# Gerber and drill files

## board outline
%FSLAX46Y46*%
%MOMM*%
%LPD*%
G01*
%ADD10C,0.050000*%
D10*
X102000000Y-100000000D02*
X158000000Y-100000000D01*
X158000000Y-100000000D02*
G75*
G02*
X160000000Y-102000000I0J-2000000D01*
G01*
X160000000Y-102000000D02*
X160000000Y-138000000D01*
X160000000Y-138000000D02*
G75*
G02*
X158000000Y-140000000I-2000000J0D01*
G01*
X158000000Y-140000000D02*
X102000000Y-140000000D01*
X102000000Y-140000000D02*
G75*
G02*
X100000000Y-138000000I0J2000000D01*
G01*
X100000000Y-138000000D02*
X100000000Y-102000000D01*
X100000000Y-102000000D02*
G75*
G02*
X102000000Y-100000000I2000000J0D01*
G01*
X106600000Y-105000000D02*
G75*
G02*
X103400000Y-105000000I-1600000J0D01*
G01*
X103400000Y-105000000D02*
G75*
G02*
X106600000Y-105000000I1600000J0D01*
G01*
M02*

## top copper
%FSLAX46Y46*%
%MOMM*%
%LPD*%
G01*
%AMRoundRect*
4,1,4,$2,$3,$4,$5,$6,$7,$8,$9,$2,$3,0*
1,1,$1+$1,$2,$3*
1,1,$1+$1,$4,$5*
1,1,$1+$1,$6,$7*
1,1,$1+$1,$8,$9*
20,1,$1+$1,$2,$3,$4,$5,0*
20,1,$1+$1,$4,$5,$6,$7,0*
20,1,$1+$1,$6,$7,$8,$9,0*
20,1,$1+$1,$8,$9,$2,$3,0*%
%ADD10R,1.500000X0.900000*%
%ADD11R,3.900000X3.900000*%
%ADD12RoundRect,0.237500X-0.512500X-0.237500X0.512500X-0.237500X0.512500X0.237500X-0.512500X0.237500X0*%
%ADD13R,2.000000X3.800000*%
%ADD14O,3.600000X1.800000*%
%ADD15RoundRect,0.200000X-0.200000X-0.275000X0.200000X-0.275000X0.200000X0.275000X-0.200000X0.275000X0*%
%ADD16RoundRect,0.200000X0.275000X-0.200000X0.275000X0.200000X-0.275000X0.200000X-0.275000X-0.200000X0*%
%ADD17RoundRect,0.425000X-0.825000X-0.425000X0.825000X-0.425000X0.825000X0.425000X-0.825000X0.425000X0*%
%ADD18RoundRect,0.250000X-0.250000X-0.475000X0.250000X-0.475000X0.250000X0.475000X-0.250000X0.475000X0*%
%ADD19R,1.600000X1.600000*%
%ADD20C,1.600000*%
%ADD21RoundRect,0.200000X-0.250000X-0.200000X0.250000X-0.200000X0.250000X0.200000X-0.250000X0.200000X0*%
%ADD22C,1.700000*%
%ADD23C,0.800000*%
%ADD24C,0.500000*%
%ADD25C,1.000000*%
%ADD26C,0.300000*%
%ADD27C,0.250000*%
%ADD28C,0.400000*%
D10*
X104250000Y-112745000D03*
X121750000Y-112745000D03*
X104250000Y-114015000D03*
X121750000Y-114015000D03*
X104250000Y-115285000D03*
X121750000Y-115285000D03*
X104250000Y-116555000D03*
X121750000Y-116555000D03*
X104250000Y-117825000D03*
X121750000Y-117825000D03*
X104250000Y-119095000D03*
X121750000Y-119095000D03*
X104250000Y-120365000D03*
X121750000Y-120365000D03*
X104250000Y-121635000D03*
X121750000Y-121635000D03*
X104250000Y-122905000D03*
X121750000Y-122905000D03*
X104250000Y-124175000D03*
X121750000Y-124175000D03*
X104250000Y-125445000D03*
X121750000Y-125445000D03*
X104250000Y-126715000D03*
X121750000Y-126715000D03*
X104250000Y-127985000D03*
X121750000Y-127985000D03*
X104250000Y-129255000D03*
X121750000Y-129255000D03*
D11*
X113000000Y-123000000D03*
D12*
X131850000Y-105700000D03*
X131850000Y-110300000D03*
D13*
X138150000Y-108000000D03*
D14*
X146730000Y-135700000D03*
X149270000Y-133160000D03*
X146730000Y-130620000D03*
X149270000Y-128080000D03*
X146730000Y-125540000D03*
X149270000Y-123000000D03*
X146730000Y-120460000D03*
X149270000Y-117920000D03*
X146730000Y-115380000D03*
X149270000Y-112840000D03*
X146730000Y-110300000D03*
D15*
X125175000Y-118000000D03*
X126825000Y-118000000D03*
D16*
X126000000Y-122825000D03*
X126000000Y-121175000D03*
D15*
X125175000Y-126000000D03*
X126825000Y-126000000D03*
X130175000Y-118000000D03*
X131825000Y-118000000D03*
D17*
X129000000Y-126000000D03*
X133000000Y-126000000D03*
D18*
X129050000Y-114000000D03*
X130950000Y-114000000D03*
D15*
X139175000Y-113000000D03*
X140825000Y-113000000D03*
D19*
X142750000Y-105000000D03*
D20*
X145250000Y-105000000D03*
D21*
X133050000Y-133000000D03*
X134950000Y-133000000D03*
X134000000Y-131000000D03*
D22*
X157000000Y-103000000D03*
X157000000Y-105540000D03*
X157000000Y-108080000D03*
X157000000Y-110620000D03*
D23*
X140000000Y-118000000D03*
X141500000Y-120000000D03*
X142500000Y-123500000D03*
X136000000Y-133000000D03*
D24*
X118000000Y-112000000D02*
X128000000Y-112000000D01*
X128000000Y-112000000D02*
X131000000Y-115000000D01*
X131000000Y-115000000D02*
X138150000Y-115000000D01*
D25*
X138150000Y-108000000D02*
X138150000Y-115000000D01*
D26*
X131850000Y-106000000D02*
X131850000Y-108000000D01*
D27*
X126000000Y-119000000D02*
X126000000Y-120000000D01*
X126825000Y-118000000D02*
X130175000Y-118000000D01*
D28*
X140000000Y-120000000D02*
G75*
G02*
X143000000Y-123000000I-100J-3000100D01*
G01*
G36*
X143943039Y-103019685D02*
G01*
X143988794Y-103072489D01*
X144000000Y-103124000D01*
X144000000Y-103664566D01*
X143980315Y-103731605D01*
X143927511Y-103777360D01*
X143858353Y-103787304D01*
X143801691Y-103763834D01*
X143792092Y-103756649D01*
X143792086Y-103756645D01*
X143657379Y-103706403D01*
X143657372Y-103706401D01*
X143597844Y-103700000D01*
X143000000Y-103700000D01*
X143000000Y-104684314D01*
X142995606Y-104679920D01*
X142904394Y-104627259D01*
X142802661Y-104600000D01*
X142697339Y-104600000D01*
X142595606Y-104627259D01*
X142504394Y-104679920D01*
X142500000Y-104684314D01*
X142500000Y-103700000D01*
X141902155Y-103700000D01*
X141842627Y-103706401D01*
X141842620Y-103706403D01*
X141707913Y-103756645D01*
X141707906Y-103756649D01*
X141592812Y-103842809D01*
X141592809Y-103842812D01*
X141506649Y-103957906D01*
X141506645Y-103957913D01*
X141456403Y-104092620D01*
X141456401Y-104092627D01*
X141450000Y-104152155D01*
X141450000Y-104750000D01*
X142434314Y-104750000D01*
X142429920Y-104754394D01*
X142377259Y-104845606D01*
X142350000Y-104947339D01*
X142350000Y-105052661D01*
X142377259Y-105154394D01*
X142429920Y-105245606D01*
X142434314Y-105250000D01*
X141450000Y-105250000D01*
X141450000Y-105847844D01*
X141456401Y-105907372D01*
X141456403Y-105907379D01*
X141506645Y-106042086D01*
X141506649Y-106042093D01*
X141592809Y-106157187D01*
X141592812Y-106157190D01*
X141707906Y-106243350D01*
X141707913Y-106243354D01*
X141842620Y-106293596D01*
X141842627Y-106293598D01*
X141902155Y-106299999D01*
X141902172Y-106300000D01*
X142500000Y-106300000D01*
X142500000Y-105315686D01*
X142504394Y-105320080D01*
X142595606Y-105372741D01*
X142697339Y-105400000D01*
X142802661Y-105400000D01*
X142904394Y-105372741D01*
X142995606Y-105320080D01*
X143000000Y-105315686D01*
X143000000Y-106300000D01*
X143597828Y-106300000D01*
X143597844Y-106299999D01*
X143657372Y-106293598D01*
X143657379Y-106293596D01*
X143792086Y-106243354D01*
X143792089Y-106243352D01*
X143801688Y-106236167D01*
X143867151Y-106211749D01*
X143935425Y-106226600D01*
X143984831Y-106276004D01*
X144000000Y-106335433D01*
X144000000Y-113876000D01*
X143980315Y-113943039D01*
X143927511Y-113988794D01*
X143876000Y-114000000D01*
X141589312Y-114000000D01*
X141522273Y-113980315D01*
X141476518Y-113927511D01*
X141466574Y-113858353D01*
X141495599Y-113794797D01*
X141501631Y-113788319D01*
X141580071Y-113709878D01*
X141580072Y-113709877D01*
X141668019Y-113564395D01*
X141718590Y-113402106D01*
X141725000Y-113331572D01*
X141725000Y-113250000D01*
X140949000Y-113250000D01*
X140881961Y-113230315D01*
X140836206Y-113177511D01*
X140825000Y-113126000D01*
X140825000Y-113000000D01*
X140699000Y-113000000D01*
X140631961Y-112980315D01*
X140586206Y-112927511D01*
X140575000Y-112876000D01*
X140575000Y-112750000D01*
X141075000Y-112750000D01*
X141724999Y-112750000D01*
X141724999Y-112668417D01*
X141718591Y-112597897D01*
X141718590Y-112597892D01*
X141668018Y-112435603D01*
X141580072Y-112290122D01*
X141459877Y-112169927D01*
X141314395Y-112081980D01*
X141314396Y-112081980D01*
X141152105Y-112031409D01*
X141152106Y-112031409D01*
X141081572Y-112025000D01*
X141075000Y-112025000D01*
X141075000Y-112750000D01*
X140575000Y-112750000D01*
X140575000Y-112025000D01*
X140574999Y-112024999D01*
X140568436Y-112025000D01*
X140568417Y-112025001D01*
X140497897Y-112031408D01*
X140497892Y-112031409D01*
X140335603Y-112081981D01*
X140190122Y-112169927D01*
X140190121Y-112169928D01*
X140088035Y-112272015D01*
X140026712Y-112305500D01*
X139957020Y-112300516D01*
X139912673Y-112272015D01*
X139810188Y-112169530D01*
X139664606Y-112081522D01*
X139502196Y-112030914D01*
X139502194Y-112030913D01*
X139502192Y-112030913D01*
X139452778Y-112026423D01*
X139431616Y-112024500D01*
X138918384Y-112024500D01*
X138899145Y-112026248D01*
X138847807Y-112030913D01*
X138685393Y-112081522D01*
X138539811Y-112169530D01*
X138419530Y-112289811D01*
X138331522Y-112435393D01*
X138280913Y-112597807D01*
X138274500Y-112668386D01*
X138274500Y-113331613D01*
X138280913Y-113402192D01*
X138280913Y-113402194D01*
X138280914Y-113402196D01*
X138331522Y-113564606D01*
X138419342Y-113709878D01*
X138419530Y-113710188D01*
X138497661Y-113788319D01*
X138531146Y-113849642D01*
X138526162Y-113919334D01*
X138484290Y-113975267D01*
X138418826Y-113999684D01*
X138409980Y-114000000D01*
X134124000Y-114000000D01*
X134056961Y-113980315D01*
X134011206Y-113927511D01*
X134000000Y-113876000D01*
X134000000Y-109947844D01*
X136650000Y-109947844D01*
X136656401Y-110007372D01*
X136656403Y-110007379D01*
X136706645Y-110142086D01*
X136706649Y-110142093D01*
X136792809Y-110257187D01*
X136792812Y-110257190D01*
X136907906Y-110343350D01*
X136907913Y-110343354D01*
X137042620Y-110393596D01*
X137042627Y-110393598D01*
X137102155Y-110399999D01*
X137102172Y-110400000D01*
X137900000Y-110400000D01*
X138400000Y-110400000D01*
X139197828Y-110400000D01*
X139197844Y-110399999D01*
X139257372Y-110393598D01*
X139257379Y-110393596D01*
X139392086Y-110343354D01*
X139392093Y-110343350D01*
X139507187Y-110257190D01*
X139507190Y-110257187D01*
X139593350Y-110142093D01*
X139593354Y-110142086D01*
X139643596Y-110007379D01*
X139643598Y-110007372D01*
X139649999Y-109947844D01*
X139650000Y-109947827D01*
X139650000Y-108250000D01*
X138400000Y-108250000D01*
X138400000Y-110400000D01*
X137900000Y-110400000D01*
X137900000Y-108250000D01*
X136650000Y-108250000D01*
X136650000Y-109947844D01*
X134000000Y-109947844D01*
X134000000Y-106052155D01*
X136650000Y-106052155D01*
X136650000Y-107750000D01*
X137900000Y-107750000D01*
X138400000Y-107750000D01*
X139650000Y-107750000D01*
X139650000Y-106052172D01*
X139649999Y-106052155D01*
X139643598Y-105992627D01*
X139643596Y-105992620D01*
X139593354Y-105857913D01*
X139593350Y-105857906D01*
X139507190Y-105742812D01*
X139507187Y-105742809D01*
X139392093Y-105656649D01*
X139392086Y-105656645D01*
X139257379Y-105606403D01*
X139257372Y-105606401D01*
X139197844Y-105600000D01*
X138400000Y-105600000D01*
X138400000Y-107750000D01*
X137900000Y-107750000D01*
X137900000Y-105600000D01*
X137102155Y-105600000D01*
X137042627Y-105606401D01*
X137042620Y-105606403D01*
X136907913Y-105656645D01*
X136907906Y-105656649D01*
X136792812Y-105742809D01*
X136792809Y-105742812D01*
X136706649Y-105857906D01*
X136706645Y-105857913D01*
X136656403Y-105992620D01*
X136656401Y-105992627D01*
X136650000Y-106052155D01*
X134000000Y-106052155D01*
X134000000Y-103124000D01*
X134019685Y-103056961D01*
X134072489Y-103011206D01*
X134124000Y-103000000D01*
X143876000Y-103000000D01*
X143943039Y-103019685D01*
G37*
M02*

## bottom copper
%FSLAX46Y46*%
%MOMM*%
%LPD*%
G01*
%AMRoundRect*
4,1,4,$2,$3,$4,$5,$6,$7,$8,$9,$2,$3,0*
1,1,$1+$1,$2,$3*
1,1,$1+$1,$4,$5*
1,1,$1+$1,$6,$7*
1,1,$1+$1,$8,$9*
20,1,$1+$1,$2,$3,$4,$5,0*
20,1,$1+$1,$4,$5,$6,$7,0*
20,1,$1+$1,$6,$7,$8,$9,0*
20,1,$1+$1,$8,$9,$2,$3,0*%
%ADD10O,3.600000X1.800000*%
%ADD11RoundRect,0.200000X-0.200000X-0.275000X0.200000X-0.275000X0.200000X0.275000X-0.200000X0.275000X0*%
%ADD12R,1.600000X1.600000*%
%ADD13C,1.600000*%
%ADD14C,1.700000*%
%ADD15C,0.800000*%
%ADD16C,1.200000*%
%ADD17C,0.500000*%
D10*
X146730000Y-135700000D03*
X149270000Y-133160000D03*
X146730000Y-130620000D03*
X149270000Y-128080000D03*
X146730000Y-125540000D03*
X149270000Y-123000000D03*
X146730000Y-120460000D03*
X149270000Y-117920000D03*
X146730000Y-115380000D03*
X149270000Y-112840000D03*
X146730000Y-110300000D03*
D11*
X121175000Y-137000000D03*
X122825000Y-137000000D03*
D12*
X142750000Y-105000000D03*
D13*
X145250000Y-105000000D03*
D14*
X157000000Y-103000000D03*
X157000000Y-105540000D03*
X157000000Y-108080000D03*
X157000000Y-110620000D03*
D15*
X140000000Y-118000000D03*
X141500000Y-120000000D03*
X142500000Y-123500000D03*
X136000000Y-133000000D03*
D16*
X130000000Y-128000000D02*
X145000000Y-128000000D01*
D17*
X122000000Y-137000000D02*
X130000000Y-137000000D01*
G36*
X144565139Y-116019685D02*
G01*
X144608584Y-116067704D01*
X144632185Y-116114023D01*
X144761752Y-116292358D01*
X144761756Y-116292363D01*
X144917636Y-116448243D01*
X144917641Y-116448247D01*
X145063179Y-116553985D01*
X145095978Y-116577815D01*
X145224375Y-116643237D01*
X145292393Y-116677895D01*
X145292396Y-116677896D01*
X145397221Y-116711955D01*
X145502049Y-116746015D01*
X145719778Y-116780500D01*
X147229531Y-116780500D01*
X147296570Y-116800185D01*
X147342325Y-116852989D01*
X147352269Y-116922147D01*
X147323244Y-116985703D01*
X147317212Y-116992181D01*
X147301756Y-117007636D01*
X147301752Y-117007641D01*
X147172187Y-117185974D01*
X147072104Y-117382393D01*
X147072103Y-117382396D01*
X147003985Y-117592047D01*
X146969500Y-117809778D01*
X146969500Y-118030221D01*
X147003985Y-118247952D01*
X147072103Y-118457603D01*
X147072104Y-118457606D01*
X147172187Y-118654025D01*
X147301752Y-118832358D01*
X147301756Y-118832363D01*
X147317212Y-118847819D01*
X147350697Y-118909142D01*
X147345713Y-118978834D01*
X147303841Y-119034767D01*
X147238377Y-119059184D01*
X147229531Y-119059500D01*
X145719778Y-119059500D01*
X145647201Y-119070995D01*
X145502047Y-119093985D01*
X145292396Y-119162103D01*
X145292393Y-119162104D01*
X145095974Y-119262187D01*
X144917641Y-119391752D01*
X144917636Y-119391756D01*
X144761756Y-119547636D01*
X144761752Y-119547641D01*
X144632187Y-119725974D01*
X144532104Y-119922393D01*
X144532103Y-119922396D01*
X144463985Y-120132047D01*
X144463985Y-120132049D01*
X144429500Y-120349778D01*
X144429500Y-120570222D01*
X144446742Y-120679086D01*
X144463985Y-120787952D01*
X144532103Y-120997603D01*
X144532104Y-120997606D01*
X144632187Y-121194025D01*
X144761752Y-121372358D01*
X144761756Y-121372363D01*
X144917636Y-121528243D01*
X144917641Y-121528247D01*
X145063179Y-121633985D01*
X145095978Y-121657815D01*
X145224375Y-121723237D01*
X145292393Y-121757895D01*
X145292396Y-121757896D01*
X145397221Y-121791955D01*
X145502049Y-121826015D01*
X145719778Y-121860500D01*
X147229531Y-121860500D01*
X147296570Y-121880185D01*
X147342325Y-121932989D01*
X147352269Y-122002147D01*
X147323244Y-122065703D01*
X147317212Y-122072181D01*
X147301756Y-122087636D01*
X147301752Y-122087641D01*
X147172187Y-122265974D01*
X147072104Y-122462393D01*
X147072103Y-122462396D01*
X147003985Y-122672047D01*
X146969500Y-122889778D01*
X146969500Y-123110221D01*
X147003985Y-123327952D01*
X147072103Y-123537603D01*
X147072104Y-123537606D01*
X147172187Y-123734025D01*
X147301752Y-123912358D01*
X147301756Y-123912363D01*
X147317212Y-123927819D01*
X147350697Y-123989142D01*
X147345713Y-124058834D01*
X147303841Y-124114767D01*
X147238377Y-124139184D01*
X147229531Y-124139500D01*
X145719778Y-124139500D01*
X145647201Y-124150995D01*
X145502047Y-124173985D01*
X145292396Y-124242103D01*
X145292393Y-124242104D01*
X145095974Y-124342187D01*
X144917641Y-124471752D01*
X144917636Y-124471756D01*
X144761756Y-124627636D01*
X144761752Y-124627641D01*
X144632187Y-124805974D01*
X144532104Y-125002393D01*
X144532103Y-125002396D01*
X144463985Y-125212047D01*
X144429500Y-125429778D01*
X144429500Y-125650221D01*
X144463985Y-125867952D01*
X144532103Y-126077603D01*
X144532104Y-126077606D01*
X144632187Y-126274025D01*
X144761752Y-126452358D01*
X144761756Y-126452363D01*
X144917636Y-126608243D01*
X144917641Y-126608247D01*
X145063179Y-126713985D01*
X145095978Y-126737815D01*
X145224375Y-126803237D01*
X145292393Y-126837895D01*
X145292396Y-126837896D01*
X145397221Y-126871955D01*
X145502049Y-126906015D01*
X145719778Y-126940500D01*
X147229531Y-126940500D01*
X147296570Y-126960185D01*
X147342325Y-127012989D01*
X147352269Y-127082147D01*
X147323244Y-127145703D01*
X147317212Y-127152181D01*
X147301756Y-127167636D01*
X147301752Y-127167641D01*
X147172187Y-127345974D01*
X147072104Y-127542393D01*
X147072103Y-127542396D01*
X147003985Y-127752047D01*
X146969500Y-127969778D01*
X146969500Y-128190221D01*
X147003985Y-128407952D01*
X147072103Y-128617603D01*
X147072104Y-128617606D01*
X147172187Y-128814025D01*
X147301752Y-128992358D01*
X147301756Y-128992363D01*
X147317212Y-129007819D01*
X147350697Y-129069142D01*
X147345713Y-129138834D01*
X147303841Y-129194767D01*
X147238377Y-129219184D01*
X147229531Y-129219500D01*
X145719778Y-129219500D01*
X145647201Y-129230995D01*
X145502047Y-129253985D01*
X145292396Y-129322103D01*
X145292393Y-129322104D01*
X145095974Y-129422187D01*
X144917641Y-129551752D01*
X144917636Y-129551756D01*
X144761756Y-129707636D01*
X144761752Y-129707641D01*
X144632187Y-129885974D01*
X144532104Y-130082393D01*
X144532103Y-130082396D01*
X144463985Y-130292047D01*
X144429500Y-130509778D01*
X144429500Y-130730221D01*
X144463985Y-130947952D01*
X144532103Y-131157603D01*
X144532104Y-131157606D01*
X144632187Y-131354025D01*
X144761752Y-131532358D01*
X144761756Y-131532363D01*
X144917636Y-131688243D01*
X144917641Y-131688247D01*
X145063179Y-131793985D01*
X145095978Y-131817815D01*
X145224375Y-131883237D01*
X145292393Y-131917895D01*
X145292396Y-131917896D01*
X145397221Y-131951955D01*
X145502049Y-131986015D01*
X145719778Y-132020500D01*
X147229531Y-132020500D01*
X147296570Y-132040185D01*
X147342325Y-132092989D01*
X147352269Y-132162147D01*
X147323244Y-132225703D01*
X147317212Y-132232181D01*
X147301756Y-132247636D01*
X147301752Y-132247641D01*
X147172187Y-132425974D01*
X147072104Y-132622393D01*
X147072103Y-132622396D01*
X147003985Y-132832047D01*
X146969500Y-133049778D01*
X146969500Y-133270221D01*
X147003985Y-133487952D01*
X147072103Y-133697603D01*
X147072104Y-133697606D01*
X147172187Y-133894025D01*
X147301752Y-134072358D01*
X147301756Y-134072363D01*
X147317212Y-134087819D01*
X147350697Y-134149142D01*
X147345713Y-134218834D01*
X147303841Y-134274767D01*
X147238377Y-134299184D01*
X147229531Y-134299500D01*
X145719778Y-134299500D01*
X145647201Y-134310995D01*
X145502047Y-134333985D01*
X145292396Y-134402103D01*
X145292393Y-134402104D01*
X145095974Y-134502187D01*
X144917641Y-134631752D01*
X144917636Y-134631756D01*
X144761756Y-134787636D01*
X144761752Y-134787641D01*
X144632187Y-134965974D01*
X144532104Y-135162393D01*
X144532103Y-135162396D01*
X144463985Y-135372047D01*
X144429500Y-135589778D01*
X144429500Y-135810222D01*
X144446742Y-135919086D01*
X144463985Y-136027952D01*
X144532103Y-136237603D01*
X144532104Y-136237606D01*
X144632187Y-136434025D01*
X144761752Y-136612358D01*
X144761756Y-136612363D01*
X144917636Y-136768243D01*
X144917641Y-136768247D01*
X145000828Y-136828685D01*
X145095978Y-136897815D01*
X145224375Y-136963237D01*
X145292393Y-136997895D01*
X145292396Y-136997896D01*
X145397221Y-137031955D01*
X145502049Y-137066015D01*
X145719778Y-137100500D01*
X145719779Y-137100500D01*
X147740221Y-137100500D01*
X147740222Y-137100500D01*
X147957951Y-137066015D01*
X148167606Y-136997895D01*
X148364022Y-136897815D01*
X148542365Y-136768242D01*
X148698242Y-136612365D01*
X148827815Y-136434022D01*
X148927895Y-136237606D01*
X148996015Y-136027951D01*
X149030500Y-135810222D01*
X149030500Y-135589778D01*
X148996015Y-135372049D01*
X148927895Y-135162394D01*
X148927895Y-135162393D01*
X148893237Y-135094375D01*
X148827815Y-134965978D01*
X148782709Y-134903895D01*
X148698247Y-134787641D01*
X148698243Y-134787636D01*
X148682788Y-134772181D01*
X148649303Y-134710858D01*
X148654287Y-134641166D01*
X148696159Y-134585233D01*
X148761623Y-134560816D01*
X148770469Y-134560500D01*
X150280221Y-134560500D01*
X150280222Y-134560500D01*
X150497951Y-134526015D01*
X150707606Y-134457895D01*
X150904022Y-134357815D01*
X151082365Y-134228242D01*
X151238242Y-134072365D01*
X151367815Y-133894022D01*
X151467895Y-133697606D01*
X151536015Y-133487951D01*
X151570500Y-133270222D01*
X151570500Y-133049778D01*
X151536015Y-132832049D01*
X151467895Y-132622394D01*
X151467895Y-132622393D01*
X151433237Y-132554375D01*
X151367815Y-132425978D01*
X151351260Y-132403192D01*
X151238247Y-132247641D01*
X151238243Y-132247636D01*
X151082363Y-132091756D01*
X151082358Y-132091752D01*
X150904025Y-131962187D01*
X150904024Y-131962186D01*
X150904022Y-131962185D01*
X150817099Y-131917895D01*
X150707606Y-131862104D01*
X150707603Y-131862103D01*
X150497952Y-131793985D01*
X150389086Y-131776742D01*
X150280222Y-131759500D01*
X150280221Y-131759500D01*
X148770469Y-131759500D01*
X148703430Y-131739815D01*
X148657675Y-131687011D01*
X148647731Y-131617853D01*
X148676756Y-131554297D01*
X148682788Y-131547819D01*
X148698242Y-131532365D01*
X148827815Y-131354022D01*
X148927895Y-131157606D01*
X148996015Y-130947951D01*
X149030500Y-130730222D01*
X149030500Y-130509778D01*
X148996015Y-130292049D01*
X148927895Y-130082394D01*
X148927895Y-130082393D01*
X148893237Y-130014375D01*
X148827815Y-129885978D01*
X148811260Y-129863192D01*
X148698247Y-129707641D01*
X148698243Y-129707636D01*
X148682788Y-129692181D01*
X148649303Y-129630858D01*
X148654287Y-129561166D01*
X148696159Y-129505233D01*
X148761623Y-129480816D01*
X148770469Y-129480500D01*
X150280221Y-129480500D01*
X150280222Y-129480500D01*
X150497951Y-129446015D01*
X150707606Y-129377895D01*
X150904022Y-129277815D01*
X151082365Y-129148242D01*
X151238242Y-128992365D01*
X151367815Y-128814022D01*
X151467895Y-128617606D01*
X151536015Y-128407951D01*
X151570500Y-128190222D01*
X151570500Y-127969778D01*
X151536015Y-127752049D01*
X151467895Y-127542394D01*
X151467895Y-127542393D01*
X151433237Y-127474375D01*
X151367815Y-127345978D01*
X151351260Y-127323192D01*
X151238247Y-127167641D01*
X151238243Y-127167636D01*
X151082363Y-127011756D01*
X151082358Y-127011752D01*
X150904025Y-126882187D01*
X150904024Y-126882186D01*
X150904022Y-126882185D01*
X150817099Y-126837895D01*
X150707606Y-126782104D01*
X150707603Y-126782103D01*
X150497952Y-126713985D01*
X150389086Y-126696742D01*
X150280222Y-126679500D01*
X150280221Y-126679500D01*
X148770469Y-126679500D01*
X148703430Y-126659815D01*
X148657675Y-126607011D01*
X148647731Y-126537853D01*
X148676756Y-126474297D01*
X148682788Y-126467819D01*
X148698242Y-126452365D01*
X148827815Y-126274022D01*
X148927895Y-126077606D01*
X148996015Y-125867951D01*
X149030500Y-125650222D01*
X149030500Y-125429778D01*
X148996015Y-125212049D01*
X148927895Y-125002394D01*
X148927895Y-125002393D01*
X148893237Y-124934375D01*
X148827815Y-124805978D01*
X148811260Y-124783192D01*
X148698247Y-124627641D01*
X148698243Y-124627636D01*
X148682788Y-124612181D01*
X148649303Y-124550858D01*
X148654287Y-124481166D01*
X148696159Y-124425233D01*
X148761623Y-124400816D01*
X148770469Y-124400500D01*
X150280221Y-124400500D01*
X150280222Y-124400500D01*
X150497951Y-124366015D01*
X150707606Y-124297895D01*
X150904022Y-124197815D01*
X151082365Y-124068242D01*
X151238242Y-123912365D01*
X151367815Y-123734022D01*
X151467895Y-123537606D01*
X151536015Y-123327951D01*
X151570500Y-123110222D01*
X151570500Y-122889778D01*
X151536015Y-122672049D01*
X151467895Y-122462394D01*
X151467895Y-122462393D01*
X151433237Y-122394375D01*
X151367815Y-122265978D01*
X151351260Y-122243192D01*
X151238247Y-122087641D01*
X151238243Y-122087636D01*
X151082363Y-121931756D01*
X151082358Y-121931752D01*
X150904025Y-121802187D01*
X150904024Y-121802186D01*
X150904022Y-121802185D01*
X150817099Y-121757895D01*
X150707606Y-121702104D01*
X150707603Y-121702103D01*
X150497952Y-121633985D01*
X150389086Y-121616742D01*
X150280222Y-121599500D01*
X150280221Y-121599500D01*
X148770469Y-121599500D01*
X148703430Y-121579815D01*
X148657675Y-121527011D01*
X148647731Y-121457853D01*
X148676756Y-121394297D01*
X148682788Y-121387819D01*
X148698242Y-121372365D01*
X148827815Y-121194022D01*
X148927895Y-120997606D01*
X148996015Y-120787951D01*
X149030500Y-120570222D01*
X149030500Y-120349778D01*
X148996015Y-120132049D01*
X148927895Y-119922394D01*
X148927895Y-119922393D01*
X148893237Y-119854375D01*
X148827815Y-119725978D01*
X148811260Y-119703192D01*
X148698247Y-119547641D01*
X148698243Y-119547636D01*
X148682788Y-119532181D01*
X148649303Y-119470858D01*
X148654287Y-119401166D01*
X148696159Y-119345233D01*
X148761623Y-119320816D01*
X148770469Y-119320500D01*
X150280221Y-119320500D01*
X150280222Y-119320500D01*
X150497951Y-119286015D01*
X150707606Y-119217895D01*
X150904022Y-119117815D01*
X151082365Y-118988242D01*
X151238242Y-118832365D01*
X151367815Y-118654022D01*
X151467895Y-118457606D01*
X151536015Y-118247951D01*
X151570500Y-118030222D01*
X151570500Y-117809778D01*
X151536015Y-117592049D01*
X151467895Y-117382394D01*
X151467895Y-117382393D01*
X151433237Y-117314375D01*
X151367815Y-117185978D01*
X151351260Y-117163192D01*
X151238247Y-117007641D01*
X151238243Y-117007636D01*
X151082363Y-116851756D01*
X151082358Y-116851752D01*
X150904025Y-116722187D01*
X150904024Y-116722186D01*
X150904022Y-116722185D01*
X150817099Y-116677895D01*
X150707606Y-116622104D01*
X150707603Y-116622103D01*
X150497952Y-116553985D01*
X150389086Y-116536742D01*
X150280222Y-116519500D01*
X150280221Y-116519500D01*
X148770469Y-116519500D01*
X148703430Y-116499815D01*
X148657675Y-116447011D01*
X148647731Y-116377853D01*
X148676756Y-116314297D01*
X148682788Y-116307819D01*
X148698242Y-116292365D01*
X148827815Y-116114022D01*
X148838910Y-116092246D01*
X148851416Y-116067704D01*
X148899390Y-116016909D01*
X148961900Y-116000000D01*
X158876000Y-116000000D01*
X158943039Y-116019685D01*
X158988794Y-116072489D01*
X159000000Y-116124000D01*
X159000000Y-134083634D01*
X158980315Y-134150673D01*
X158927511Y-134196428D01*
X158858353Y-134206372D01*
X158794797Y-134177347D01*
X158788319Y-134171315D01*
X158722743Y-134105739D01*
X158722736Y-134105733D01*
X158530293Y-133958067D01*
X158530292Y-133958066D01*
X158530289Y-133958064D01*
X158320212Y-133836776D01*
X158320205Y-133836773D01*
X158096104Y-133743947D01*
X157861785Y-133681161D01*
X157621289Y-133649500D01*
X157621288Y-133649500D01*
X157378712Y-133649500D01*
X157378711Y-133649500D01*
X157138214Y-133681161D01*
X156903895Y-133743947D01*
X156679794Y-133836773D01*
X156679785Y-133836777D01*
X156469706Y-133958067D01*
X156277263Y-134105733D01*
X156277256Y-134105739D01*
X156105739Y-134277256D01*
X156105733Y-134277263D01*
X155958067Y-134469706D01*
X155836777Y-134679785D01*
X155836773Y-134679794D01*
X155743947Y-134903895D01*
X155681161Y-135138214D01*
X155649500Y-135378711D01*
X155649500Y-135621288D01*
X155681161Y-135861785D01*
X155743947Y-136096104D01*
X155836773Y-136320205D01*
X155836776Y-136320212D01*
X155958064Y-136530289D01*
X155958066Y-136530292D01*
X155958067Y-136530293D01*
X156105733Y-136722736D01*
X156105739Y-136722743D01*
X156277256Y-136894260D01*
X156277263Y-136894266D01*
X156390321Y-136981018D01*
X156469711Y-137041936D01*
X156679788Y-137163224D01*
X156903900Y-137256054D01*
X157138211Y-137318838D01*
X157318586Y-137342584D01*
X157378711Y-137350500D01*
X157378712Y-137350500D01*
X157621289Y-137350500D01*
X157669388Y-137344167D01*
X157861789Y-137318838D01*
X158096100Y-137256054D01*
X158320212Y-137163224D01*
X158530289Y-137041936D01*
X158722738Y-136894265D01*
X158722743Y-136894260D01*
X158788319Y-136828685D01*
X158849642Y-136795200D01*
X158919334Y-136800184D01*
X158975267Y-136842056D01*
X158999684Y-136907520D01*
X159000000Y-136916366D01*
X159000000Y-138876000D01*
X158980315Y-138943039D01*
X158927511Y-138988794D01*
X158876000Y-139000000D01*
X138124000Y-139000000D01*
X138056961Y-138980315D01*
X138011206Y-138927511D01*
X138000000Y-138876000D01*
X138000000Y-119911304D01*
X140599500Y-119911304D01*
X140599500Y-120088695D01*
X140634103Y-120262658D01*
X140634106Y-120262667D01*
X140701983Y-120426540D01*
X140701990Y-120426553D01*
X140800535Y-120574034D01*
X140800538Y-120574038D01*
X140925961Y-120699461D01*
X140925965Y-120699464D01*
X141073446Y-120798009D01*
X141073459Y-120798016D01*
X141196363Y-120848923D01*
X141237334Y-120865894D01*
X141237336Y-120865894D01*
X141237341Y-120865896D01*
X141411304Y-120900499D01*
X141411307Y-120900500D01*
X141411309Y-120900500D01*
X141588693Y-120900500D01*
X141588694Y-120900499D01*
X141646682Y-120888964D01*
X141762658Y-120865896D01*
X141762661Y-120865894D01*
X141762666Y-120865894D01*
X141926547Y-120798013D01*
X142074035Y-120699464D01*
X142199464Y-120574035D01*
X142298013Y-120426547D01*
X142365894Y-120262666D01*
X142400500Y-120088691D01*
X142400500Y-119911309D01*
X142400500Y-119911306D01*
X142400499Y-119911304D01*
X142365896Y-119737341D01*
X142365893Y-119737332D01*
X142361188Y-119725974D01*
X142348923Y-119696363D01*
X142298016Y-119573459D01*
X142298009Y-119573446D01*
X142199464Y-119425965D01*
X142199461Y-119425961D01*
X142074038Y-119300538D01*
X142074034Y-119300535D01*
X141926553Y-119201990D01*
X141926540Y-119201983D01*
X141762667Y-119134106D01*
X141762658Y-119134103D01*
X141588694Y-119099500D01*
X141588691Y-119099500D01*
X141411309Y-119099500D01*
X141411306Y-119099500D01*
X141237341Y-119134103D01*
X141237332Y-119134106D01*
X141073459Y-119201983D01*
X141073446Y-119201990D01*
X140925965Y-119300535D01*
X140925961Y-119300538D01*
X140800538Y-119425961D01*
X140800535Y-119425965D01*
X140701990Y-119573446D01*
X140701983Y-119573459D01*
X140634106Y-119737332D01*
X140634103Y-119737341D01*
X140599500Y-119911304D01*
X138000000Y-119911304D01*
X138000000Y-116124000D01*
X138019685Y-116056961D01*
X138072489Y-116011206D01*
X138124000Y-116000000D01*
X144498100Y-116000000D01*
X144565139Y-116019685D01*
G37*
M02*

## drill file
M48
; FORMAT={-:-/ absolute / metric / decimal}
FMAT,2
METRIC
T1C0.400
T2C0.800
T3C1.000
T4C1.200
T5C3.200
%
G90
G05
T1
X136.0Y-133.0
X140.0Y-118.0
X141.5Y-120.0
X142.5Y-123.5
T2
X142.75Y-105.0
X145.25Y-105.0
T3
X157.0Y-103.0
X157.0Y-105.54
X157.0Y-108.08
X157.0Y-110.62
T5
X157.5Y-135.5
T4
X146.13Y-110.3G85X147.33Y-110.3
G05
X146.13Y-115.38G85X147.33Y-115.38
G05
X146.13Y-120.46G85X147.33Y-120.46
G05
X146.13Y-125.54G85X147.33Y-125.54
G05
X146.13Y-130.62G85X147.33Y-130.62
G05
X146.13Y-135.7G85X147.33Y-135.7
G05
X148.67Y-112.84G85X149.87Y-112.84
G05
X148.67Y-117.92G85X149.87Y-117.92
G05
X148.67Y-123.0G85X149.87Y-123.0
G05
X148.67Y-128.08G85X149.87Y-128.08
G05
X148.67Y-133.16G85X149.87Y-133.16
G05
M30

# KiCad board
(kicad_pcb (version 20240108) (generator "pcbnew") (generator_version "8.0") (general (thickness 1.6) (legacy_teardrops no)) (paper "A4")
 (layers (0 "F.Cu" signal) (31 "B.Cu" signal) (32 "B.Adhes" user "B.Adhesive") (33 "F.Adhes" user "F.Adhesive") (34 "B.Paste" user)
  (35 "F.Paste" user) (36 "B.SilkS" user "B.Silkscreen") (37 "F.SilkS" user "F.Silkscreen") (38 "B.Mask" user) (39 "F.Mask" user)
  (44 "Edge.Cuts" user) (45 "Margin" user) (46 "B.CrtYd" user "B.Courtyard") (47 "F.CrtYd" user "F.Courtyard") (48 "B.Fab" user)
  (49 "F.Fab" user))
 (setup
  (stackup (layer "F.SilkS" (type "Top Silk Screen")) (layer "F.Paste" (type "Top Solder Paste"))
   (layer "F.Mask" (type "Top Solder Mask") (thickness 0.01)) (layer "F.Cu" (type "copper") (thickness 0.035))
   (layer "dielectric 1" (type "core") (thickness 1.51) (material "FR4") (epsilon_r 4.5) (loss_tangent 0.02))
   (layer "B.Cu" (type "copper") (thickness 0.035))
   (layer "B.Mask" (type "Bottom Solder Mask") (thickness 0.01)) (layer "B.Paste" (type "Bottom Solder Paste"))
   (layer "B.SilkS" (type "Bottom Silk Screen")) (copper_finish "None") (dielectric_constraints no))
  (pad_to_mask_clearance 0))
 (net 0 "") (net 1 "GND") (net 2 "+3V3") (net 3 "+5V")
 (gr_line (start 102 100) (end 158 100) (stroke (width 0.05) (type default)) (layer "Edge.Cuts"))
 (gr_arc (start 158 100) (mid 159.4142 100.5858) (end 160 102) (stroke (width 0.05) (type default)) (layer "Edge.Cuts"))
 (gr_line (start 160 102) (end 160 138) (stroke (width 0.05) (type default)) (layer "Edge.Cuts"))
 (gr_arc (start 160 138) (mid 159.4142 139.4142) (end 158 140) (stroke (width 0.05) (type default)) (layer "Edge.Cuts"))
 (gr_line (start 158 140) (end 102 140) (stroke (width 0.05) (type default)) (layer "Edge.Cuts"))
 (gr_arc (start 102 140) (mid 100.5858 139.4142) (end 100 138) (stroke (width 0.05) (type default)) (layer "Edge.Cuts"))
 (gr_line (start 100 138) (end 100 102) (stroke (width 0.05) (type default)) (layer "Edge.Cuts"))
 (gr_arc (start 100 102) (mid 100.5858 100.5858) (end 102 100) (stroke (width 0.05) (type default)) (layer "Edge.Cuts"))
 (gr_circle (center 105 105) (end 106.6 105) (stroke (width 0.05) (type default)) (fill none) (layer "Edge.Cuts"))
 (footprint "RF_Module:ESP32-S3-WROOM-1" (layer "F.Cu") (at 113 121)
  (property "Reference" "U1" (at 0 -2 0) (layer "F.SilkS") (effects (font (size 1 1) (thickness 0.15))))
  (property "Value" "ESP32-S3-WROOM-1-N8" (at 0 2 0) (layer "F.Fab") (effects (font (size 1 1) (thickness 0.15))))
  (pad "1" smd rect (at -8.75 -8.255) (size 1.5 0.9) (layers "F.Cu" "F.Paste" "F.Mask") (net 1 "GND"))
  (pad "15" smd rect (at 8.75 -8.255) (size 1.5 0.9) (layers "F.Cu" "F.Paste" "F.Mask") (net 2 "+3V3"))
  (pad "2" smd rect (at -8.75 -6.985) (size 1.5 0.9) (layers "F.Cu" "F.Paste" "F.Mask"))
  (pad "16" smd rect (at 8.75 -6.985) (size 1.5 0.9) (layers "F.Cu" "F.Paste" "F.Mask"))
  (pad "3" smd rect (at -8.75 -5.715) (size 1.5 0.9) (layers "F.Cu" "F.Paste" "F.Mask"))
  (pad "17" smd rect (at 8.75 -5.715) (size 1.5 0.9) (layers "F.Cu" "F.Paste" "F.Mask"))
  (pad "4" smd rect (at -8.75 -4.445) (size 1.5 0.9) (layers "F.Cu" "F.Paste" "F.Mask"))
  (pad "18" smd rect (at 8.75 -4.445) (size 1.5 0.9) (layers "F.Cu" "F.Paste" "F.Mask"))
  (pad "5" smd rect (at -8.75 -3.175) (size 1.5 0.9) (layers "F.Cu" "F.Paste" "F.Mask"))
  (pad "19" smd rect (at 8.75 -3.175) (size 1.5 0.9) (layers "F.Cu" "F.Paste" "F.Mask"))
  (pad "6" smd rect (at -8.75 -1.905) (size 1.5 0.9) (layers "F.Cu" "F.Paste" "F.Mask"))
  (pad "20" smd rect (at 8.75 -1.905) (size 1.5 0.9) (layers "F.Cu" "F.Paste" "F.Mask"))
  (pad "7" smd rect (at -8.75 -0.635) (size 1.5 0.9) (layers "F.Cu" "F.Paste" "F.Mask"))
  (pad "21" smd rect (at 8.75 -0.635) (size 1.5 0.9) (layers "F.Cu" "F.Paste" "F.Mask"))
  (pad "8" smd rect (at -8.75 0.635) (size 1.5 0.9) (layers "F.Cu" "F.Paste" "F.Mask"))
  (pad "22" smd rect (at 8.75 0.635) (size 1.5 0.9) (layers "F.Cu" "F.Paste" "F.Mask"))
  (pad "9" smd rect (at -8.75 1.905) (size 1.5 0.9) (layers "F.Cu" "F.Paste" "F.Mask"))
  (pad "23" smd rect (at 8.75 1.905) (size 1.5 0.9) (layers "F.Cu" "F.Paste" "F.Mask"))
  (pad "10" smd rect (at -8.75 3.175) (size 1.5 0.9) (layers "F.Cu" "F.Paste" "F.Mask"))
  (pad "24" smd rect (at 8.75 3.175) (size 1.5 0.9) (layers "F.Cu" "F.Paste" "F.Mask"))
  (pad "11" smd rect (at -8.75 4.445) (size 1.5 0.9) (layers "F.Cu" "F.Paste" "F.Mask"))
  (pad "25" smd rect (at 8.75 4.445) (size 1.5 0.9) (layers "F.Cu" "F.Paste" "F.Mask"))
  (pad "12" smd rect (at -8.75 5.715) (size 1.5 0.9) (layers "F.Cu" "F.Paste" "F.Mask"))
  (pad "26" smd rect (at 8.75 5.715) (size 1.5 0.9) (layers "F.Cu" "F.Paste" "F.Mask"))
  (pad "13" smd rect (at -8.75 6.985) (size 1.5 0.9) (layers "F.Cu" "F.Paste" "F.Mask"))
  (pad "27" smd rect (at 8.75 6.985) (size 1.5 0.9) (layers "F.Cu" "F.Paste" "F.Mask"))
  (pad "14" smd rect (at -8.75 8.255) (size 1.5 0.9) (layers "F.Cu" "F.Paste" "F.Mask") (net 1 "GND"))
  (pad "28" smd rect (at 8.75 8.255) (size 1.5 0.9) (layers "F.Cu" "F.Paste" "F.Mask"))
  (pad "41" smd rect (at 0 2) (size 3.9 3.9) (layers "F.Cu" "F.Paste" "F.Mask") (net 1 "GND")))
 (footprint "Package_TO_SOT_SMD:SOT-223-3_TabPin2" (layer "F.Cu") (at 135 108)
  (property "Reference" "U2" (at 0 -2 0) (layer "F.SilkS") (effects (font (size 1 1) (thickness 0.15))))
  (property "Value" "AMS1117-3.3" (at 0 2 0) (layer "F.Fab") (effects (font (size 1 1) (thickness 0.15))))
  (pad "1" smd roundrect (at -3.15 -2.3) (size 1.5 0.95) (layers "F.Cu" "F.Paste" "F.Mask") (roundrect_rratio 0.25) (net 1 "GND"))
  (pad "3" smd roundrect (at -3.15 2.3) (size 1.5 0.95) (layers "F.Cu" "F.Paste" "F.Mask") (roundrect_rratio 0.25) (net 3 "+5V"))
  (pad "2" smd rect (at 3.15 0) (size 2 3.8) (layers "F.Cu" "F.Paste" "F.Mask") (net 2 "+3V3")))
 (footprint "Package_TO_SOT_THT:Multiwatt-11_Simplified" (layer "F.Cu") (at 148 123 90)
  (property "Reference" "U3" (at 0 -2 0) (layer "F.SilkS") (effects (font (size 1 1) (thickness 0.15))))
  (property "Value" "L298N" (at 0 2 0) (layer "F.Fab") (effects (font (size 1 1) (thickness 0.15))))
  (pad "1" thru_hole oval (at -12.7 -1.27 90) (size 1.8 3.6) (drill oval 1.2 2.4) (layers "*.Cu" "*.Mask"))
  (pad "2" thru_hole oval (at -10.16 1.27 90) (size 1.8 3.6) (drill oval 1.2 2.4) (layers "*.Cu" "*.Mask"))
  (pad "3" thru_hole oval (at -7.62 -1.27 90) (size 1.8 3.6) (drill oval 1.2 2.4) (layers "*.Cu" "*.Mask"))
  (pad "4" thru_hole oval (at -5.08 1.27 90) (size 1.8 3.6) (drill oval 1.2 2.4) (layers "*.Cu" "*.Mask") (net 3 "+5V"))
  (pad "5" thru_hole oval (at -2.54 -1.27 90) (size 1.8 3.6) (drill oval 1.2 2.4) (layers "*.Cu" "*.Mask"))
  (pad "6" thru_hole oval (at 0 1.27 90) (size 1.8 3.6) (drill oval 1.2 2.4) (layers "*.Cu" "*.Mask"))
  (pad "7" thru_hole oval (at 2.54 -1.27 90) (size 1.8 3.6) (drill oval 1.2 2.4) (layers "*.Cu" "*.Mask"))
  (pad "8" thru_hole oval (at 5.08 1.27 90) (size 1.8 3.6) (drill oval 1.2 2.4) (layers "*.Cu" "*.Mask"))
  (pad "9" thru_hole oval (at 7.62 -1.27 90) (size 1.8 3.6) (drill oval 1.2 2.4) (layers "*.Cu" "*.Mask"))
  (pad "10" thru_hole oval (at 10.16 1.27 90) (size 1.8 3.6) (drill oval 1.2 2.4) (layers "*.Cu" "*.Mask"))
  (pad "11" thru_hole oval (at 12.7 -1.27 90) (size 1.8 3.6) (drill oval 1.2 2.4) (layers "*.Cu" "*.Mask")))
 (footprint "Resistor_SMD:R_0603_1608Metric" (layer "F.Cu") (at 126 118)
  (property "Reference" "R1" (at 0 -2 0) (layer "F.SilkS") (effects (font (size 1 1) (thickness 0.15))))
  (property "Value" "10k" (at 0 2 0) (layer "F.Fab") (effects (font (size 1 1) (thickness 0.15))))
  (pad "1" smd roundrect (at -0.825 0) (size 0.8 0.95) (layers "F.Cu" "F.Paste" "F.Mask") (roundrect_rratio 0.25) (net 1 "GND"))
  (pad "2" smd roundrect (at 0.825 0) (size 0.8 0.95) (layers "F.Cu" "F.Paste" "F.Mask") (roundrect_rratio 0.25) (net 2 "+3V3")))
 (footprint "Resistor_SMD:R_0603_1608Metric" (layer "F.Cu") (at 126 122 90)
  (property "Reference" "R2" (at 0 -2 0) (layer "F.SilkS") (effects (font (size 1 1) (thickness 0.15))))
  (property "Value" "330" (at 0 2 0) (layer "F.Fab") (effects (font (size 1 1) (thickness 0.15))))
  (pad "1" smd roundrect (at -0.825 0 90) (size 0.8 0.95) (layers "F.Cu" "F.Paste" "F.Mask") (roundrect_rratio 0.25) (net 1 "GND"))
  (pad "2" smd roundrect (at 0.825 0 90) (size 0.8 0.95) (layers "F.Cu" "F.Paste" "F.Mask") (roundrect_rratio 0.25) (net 2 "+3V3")))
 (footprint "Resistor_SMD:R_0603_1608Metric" (layer "F.Cu") (at 126 126)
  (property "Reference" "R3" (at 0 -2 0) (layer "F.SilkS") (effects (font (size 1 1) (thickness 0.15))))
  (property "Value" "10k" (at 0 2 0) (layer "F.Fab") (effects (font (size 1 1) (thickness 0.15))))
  (pad "1" smd roundrect (at -0.825 0) (size 0.8 0.95) (layers "F.Cu" "F.Paste" "F.Mask") (roundrect_rratio 0.25) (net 1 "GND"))
  (pad "2" smd roundrect (at 0.825 0) (size 0.8 0.95) (layers "F.Cu" "F.Paste" "F.Mask") (roundrect_rratio 0.25) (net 2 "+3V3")))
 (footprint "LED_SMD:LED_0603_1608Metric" (layer "F.Cu") (at 131 118)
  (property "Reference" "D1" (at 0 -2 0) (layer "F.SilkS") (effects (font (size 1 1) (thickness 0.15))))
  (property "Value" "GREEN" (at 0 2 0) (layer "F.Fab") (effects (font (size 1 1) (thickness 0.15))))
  (pad "1" smd roundrect (at -0.825 0) (size 0.8 0.95) (layers "F.Cu" "F.Paste" "F.Mask") (roundrect_rratio 0.25) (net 1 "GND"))
  (pad "2" smd roundrect (at 0.825 0) (size 0.8 0.95) (layers "F.Cu" "F.Paste" "F.Mask") (roundrect_rratio 0.25) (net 2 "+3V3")))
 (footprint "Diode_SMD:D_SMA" (layer "F.Cu") (at 131 126)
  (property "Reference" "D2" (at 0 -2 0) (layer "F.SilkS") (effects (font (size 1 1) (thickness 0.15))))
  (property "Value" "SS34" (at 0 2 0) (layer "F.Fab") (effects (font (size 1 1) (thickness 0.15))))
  (pad "1" smd roundrect (at -2 0) (size 2.5 1.7) (layers "F.Cu" "F.Paste" "F.Mask") (roundrect_rratio 0.25) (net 1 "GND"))
  (pad "2" smd roundrect (at 2 0) (size 2.5 1.7) (layers "F.Cu" "F.Paste" "F.Mask") (roundrect_rratio 0.25) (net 2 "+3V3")))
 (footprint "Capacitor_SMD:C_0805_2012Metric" (layer "F.Cu") (at 130 114)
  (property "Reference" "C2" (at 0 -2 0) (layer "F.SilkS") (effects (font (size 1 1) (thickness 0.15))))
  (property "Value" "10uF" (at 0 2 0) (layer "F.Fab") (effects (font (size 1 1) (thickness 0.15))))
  (pad "1" smd roundrect (at -0.95 0) (size 1 1.45) (layers "F.Cu" "F.Paste" "F.Mask") (roundrect_rratio 0.25) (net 1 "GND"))
  (pad "2" smd roundrect (at 0.95 0) (size 1 1.45) (layers "F.Cu" "F.Paste" "F.Mask") (roundrect_rratio 0.25) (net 2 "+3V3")))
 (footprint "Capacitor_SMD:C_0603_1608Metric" (layer "F.Cu") (at 140 113)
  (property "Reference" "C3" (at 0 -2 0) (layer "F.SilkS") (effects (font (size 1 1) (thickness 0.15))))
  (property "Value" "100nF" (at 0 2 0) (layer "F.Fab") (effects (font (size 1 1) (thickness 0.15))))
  (pad "1" smd roundrect (at -0.825 0) (size 0.8 0.95) (layers "F.Cu" "F.Paste" "F.Mask") (roundrect_rratio 0.25) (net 1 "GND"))
  (pad "2" smd roundrect (at 0.825 0) (size 0.8 0.95) (layers "F.Cu" "F.Paste" "F.Mask") (roundrect_rratio 0.25) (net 2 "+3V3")))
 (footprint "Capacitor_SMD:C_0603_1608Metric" (layer "B.Cu") (at 122 137)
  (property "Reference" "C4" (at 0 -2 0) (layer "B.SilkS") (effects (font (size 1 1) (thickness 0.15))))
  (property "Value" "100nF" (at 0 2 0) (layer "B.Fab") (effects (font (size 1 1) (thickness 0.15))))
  (pad "1" smd roundrect (at -0.825 0) (size 0.8 0.95) (layers "B.Cu" "B.Paste" "B.Mask") (roundrect_rratio 0.25) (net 1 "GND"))
  (pad "2" smd roundrect (at 0.825 0) (size 0.8 0.95) (layers "B.Cu" "B.Paste" "B.Mask") (roundrect_rratio 0.25) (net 2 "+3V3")))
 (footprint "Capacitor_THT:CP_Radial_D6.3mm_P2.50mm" (layer "F.Cu") (at 144 105)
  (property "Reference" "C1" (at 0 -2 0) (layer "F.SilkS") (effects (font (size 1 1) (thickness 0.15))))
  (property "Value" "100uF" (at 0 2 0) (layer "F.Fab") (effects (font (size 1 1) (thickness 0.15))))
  (pad "1" thru_hole rect (at -1.25 0) (size 1.6 1.6) (drill 0.8) (layers "*.Cu" "*.Mask") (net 2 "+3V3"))
  (pad "2" thru_hole circle (at 1.25 0) (size 1.6 1.6) (drill 0.8) (layers "*.Cu" "*.Mask") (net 1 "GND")))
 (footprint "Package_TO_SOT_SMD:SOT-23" (layer "F.Cu") (at 134 132)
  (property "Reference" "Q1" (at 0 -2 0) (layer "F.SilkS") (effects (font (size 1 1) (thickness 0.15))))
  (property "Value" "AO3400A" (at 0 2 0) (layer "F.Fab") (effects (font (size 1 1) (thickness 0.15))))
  (pad "1" smd roundrect (at -0.95 1) (size 0.9 0.8) (layers "F.Cu" "F.Paste" "F.Mask") (roundrect_rratio 0.25))
  (pad "2" smd roundrect (at 0.95 1) (size 0.9 0.8) (layers "F.Cu" "F.Paste" "F.Mask") (roundrect_rratio 0.25))
  (pad "3" smd roundrect (at 0 -1) (size 0.9 0.8) (layers "F.Cu" "F.Paste" "F.Mask") (roundrect_rratio 0.25)))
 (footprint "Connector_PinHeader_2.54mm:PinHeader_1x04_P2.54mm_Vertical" (layer "F.Cu") (at 157 103)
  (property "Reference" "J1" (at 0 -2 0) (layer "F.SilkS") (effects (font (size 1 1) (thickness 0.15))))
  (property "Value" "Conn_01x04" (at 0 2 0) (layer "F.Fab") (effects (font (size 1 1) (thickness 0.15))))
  (pad "1" thru_hole circle (at 0 0) (size 1.7 1.7) (drill 1) (layers "*.Cu" "*.Mask"))
  (pad "2" thru_hole circle (at 0 2.54) (size 1.7 1.7) (drill 1) (layers "*.Cu" "*.Mask"))
  (pad "3" thru_hole circle (at 0 5.08) (size 1.7 1.7) (drill 1) (layers "*.Cu" "*.Mask"))
  (pad "4" thru_hole circle (at 0 7.62) (size 1.7 1.7) (drill 1) (layers "*.Cu" "*.Mask")))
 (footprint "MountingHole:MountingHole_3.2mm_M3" (layer "F.Cu") (at 157.5 135.5)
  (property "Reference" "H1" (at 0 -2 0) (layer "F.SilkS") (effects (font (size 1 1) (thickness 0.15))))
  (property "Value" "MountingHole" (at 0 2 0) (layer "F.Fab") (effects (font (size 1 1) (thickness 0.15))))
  (pad "1" np_thru_hole circle (at 0 0) (size 3.2 3.2) (drill 3.2) (layers "*.Cu" "*.Mask")))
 (segment (start 118 112) (end 128 112) (width 0.5) (layer "F.Cu") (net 2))
 (segment (start 128 112) (end 131 115) (width 0.5) (layer "F.Cu") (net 2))
 (segment (start 131 115) (end 138.15 115) (width 0.5) (layer "F.Cu") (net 2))
 (segment (start 138.15 108) (end 138.15 115) (width 1) (layer "F.Cu") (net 2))
 (segment (start 131.85 106) (end 131.85 108) (width 0.3) (layer "F.Cu") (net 1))
 (segment (start 126 119) (end 126 120) (width 0.25) (layer "F.Cu") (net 1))
 (segment (start 126.825 118) (end 130.175 118) (width 0.25) (layer "F.Cu") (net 1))
 (segment (start 130 128) (end 145 128) (width 1.2) (layer "B.Cu") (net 1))
 (segment (start 122 137) (end 130 137) (width 0.5) (layer "B.Cu") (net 1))
 (arc (start 140 120) (mid 142.1213 120.8787) (end 143 123) (width 0.4) (layer "F.Cu") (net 3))
 (via (at 140 118) (size 0.8) (drill 0.4) (layers "F.Cu" "B.Cu") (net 1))
 (via (at 141.5 120) (size 0.8) (drill 0.4) (layers "F.Cu" "B.Cu") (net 1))
 (via (at 142.5 123.5) (size 0.8) (drill 0.4) (layers "F.Cu" "B.Cu") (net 1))
 (via (at 136 133) (size 0.8) (drill 0.4) (layers "F.Cu" "B.Cu") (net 1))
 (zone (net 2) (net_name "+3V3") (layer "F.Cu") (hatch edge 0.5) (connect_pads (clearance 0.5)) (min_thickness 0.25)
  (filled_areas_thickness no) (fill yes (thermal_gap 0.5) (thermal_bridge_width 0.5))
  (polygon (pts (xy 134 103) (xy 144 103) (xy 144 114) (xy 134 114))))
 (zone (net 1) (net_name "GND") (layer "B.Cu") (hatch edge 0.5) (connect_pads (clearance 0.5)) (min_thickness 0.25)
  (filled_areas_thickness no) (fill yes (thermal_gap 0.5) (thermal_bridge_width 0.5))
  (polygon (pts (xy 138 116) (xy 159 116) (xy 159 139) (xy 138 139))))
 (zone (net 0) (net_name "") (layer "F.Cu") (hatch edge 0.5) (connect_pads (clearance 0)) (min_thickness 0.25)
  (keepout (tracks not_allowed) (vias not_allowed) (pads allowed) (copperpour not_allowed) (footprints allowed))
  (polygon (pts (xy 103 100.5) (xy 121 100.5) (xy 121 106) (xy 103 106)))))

